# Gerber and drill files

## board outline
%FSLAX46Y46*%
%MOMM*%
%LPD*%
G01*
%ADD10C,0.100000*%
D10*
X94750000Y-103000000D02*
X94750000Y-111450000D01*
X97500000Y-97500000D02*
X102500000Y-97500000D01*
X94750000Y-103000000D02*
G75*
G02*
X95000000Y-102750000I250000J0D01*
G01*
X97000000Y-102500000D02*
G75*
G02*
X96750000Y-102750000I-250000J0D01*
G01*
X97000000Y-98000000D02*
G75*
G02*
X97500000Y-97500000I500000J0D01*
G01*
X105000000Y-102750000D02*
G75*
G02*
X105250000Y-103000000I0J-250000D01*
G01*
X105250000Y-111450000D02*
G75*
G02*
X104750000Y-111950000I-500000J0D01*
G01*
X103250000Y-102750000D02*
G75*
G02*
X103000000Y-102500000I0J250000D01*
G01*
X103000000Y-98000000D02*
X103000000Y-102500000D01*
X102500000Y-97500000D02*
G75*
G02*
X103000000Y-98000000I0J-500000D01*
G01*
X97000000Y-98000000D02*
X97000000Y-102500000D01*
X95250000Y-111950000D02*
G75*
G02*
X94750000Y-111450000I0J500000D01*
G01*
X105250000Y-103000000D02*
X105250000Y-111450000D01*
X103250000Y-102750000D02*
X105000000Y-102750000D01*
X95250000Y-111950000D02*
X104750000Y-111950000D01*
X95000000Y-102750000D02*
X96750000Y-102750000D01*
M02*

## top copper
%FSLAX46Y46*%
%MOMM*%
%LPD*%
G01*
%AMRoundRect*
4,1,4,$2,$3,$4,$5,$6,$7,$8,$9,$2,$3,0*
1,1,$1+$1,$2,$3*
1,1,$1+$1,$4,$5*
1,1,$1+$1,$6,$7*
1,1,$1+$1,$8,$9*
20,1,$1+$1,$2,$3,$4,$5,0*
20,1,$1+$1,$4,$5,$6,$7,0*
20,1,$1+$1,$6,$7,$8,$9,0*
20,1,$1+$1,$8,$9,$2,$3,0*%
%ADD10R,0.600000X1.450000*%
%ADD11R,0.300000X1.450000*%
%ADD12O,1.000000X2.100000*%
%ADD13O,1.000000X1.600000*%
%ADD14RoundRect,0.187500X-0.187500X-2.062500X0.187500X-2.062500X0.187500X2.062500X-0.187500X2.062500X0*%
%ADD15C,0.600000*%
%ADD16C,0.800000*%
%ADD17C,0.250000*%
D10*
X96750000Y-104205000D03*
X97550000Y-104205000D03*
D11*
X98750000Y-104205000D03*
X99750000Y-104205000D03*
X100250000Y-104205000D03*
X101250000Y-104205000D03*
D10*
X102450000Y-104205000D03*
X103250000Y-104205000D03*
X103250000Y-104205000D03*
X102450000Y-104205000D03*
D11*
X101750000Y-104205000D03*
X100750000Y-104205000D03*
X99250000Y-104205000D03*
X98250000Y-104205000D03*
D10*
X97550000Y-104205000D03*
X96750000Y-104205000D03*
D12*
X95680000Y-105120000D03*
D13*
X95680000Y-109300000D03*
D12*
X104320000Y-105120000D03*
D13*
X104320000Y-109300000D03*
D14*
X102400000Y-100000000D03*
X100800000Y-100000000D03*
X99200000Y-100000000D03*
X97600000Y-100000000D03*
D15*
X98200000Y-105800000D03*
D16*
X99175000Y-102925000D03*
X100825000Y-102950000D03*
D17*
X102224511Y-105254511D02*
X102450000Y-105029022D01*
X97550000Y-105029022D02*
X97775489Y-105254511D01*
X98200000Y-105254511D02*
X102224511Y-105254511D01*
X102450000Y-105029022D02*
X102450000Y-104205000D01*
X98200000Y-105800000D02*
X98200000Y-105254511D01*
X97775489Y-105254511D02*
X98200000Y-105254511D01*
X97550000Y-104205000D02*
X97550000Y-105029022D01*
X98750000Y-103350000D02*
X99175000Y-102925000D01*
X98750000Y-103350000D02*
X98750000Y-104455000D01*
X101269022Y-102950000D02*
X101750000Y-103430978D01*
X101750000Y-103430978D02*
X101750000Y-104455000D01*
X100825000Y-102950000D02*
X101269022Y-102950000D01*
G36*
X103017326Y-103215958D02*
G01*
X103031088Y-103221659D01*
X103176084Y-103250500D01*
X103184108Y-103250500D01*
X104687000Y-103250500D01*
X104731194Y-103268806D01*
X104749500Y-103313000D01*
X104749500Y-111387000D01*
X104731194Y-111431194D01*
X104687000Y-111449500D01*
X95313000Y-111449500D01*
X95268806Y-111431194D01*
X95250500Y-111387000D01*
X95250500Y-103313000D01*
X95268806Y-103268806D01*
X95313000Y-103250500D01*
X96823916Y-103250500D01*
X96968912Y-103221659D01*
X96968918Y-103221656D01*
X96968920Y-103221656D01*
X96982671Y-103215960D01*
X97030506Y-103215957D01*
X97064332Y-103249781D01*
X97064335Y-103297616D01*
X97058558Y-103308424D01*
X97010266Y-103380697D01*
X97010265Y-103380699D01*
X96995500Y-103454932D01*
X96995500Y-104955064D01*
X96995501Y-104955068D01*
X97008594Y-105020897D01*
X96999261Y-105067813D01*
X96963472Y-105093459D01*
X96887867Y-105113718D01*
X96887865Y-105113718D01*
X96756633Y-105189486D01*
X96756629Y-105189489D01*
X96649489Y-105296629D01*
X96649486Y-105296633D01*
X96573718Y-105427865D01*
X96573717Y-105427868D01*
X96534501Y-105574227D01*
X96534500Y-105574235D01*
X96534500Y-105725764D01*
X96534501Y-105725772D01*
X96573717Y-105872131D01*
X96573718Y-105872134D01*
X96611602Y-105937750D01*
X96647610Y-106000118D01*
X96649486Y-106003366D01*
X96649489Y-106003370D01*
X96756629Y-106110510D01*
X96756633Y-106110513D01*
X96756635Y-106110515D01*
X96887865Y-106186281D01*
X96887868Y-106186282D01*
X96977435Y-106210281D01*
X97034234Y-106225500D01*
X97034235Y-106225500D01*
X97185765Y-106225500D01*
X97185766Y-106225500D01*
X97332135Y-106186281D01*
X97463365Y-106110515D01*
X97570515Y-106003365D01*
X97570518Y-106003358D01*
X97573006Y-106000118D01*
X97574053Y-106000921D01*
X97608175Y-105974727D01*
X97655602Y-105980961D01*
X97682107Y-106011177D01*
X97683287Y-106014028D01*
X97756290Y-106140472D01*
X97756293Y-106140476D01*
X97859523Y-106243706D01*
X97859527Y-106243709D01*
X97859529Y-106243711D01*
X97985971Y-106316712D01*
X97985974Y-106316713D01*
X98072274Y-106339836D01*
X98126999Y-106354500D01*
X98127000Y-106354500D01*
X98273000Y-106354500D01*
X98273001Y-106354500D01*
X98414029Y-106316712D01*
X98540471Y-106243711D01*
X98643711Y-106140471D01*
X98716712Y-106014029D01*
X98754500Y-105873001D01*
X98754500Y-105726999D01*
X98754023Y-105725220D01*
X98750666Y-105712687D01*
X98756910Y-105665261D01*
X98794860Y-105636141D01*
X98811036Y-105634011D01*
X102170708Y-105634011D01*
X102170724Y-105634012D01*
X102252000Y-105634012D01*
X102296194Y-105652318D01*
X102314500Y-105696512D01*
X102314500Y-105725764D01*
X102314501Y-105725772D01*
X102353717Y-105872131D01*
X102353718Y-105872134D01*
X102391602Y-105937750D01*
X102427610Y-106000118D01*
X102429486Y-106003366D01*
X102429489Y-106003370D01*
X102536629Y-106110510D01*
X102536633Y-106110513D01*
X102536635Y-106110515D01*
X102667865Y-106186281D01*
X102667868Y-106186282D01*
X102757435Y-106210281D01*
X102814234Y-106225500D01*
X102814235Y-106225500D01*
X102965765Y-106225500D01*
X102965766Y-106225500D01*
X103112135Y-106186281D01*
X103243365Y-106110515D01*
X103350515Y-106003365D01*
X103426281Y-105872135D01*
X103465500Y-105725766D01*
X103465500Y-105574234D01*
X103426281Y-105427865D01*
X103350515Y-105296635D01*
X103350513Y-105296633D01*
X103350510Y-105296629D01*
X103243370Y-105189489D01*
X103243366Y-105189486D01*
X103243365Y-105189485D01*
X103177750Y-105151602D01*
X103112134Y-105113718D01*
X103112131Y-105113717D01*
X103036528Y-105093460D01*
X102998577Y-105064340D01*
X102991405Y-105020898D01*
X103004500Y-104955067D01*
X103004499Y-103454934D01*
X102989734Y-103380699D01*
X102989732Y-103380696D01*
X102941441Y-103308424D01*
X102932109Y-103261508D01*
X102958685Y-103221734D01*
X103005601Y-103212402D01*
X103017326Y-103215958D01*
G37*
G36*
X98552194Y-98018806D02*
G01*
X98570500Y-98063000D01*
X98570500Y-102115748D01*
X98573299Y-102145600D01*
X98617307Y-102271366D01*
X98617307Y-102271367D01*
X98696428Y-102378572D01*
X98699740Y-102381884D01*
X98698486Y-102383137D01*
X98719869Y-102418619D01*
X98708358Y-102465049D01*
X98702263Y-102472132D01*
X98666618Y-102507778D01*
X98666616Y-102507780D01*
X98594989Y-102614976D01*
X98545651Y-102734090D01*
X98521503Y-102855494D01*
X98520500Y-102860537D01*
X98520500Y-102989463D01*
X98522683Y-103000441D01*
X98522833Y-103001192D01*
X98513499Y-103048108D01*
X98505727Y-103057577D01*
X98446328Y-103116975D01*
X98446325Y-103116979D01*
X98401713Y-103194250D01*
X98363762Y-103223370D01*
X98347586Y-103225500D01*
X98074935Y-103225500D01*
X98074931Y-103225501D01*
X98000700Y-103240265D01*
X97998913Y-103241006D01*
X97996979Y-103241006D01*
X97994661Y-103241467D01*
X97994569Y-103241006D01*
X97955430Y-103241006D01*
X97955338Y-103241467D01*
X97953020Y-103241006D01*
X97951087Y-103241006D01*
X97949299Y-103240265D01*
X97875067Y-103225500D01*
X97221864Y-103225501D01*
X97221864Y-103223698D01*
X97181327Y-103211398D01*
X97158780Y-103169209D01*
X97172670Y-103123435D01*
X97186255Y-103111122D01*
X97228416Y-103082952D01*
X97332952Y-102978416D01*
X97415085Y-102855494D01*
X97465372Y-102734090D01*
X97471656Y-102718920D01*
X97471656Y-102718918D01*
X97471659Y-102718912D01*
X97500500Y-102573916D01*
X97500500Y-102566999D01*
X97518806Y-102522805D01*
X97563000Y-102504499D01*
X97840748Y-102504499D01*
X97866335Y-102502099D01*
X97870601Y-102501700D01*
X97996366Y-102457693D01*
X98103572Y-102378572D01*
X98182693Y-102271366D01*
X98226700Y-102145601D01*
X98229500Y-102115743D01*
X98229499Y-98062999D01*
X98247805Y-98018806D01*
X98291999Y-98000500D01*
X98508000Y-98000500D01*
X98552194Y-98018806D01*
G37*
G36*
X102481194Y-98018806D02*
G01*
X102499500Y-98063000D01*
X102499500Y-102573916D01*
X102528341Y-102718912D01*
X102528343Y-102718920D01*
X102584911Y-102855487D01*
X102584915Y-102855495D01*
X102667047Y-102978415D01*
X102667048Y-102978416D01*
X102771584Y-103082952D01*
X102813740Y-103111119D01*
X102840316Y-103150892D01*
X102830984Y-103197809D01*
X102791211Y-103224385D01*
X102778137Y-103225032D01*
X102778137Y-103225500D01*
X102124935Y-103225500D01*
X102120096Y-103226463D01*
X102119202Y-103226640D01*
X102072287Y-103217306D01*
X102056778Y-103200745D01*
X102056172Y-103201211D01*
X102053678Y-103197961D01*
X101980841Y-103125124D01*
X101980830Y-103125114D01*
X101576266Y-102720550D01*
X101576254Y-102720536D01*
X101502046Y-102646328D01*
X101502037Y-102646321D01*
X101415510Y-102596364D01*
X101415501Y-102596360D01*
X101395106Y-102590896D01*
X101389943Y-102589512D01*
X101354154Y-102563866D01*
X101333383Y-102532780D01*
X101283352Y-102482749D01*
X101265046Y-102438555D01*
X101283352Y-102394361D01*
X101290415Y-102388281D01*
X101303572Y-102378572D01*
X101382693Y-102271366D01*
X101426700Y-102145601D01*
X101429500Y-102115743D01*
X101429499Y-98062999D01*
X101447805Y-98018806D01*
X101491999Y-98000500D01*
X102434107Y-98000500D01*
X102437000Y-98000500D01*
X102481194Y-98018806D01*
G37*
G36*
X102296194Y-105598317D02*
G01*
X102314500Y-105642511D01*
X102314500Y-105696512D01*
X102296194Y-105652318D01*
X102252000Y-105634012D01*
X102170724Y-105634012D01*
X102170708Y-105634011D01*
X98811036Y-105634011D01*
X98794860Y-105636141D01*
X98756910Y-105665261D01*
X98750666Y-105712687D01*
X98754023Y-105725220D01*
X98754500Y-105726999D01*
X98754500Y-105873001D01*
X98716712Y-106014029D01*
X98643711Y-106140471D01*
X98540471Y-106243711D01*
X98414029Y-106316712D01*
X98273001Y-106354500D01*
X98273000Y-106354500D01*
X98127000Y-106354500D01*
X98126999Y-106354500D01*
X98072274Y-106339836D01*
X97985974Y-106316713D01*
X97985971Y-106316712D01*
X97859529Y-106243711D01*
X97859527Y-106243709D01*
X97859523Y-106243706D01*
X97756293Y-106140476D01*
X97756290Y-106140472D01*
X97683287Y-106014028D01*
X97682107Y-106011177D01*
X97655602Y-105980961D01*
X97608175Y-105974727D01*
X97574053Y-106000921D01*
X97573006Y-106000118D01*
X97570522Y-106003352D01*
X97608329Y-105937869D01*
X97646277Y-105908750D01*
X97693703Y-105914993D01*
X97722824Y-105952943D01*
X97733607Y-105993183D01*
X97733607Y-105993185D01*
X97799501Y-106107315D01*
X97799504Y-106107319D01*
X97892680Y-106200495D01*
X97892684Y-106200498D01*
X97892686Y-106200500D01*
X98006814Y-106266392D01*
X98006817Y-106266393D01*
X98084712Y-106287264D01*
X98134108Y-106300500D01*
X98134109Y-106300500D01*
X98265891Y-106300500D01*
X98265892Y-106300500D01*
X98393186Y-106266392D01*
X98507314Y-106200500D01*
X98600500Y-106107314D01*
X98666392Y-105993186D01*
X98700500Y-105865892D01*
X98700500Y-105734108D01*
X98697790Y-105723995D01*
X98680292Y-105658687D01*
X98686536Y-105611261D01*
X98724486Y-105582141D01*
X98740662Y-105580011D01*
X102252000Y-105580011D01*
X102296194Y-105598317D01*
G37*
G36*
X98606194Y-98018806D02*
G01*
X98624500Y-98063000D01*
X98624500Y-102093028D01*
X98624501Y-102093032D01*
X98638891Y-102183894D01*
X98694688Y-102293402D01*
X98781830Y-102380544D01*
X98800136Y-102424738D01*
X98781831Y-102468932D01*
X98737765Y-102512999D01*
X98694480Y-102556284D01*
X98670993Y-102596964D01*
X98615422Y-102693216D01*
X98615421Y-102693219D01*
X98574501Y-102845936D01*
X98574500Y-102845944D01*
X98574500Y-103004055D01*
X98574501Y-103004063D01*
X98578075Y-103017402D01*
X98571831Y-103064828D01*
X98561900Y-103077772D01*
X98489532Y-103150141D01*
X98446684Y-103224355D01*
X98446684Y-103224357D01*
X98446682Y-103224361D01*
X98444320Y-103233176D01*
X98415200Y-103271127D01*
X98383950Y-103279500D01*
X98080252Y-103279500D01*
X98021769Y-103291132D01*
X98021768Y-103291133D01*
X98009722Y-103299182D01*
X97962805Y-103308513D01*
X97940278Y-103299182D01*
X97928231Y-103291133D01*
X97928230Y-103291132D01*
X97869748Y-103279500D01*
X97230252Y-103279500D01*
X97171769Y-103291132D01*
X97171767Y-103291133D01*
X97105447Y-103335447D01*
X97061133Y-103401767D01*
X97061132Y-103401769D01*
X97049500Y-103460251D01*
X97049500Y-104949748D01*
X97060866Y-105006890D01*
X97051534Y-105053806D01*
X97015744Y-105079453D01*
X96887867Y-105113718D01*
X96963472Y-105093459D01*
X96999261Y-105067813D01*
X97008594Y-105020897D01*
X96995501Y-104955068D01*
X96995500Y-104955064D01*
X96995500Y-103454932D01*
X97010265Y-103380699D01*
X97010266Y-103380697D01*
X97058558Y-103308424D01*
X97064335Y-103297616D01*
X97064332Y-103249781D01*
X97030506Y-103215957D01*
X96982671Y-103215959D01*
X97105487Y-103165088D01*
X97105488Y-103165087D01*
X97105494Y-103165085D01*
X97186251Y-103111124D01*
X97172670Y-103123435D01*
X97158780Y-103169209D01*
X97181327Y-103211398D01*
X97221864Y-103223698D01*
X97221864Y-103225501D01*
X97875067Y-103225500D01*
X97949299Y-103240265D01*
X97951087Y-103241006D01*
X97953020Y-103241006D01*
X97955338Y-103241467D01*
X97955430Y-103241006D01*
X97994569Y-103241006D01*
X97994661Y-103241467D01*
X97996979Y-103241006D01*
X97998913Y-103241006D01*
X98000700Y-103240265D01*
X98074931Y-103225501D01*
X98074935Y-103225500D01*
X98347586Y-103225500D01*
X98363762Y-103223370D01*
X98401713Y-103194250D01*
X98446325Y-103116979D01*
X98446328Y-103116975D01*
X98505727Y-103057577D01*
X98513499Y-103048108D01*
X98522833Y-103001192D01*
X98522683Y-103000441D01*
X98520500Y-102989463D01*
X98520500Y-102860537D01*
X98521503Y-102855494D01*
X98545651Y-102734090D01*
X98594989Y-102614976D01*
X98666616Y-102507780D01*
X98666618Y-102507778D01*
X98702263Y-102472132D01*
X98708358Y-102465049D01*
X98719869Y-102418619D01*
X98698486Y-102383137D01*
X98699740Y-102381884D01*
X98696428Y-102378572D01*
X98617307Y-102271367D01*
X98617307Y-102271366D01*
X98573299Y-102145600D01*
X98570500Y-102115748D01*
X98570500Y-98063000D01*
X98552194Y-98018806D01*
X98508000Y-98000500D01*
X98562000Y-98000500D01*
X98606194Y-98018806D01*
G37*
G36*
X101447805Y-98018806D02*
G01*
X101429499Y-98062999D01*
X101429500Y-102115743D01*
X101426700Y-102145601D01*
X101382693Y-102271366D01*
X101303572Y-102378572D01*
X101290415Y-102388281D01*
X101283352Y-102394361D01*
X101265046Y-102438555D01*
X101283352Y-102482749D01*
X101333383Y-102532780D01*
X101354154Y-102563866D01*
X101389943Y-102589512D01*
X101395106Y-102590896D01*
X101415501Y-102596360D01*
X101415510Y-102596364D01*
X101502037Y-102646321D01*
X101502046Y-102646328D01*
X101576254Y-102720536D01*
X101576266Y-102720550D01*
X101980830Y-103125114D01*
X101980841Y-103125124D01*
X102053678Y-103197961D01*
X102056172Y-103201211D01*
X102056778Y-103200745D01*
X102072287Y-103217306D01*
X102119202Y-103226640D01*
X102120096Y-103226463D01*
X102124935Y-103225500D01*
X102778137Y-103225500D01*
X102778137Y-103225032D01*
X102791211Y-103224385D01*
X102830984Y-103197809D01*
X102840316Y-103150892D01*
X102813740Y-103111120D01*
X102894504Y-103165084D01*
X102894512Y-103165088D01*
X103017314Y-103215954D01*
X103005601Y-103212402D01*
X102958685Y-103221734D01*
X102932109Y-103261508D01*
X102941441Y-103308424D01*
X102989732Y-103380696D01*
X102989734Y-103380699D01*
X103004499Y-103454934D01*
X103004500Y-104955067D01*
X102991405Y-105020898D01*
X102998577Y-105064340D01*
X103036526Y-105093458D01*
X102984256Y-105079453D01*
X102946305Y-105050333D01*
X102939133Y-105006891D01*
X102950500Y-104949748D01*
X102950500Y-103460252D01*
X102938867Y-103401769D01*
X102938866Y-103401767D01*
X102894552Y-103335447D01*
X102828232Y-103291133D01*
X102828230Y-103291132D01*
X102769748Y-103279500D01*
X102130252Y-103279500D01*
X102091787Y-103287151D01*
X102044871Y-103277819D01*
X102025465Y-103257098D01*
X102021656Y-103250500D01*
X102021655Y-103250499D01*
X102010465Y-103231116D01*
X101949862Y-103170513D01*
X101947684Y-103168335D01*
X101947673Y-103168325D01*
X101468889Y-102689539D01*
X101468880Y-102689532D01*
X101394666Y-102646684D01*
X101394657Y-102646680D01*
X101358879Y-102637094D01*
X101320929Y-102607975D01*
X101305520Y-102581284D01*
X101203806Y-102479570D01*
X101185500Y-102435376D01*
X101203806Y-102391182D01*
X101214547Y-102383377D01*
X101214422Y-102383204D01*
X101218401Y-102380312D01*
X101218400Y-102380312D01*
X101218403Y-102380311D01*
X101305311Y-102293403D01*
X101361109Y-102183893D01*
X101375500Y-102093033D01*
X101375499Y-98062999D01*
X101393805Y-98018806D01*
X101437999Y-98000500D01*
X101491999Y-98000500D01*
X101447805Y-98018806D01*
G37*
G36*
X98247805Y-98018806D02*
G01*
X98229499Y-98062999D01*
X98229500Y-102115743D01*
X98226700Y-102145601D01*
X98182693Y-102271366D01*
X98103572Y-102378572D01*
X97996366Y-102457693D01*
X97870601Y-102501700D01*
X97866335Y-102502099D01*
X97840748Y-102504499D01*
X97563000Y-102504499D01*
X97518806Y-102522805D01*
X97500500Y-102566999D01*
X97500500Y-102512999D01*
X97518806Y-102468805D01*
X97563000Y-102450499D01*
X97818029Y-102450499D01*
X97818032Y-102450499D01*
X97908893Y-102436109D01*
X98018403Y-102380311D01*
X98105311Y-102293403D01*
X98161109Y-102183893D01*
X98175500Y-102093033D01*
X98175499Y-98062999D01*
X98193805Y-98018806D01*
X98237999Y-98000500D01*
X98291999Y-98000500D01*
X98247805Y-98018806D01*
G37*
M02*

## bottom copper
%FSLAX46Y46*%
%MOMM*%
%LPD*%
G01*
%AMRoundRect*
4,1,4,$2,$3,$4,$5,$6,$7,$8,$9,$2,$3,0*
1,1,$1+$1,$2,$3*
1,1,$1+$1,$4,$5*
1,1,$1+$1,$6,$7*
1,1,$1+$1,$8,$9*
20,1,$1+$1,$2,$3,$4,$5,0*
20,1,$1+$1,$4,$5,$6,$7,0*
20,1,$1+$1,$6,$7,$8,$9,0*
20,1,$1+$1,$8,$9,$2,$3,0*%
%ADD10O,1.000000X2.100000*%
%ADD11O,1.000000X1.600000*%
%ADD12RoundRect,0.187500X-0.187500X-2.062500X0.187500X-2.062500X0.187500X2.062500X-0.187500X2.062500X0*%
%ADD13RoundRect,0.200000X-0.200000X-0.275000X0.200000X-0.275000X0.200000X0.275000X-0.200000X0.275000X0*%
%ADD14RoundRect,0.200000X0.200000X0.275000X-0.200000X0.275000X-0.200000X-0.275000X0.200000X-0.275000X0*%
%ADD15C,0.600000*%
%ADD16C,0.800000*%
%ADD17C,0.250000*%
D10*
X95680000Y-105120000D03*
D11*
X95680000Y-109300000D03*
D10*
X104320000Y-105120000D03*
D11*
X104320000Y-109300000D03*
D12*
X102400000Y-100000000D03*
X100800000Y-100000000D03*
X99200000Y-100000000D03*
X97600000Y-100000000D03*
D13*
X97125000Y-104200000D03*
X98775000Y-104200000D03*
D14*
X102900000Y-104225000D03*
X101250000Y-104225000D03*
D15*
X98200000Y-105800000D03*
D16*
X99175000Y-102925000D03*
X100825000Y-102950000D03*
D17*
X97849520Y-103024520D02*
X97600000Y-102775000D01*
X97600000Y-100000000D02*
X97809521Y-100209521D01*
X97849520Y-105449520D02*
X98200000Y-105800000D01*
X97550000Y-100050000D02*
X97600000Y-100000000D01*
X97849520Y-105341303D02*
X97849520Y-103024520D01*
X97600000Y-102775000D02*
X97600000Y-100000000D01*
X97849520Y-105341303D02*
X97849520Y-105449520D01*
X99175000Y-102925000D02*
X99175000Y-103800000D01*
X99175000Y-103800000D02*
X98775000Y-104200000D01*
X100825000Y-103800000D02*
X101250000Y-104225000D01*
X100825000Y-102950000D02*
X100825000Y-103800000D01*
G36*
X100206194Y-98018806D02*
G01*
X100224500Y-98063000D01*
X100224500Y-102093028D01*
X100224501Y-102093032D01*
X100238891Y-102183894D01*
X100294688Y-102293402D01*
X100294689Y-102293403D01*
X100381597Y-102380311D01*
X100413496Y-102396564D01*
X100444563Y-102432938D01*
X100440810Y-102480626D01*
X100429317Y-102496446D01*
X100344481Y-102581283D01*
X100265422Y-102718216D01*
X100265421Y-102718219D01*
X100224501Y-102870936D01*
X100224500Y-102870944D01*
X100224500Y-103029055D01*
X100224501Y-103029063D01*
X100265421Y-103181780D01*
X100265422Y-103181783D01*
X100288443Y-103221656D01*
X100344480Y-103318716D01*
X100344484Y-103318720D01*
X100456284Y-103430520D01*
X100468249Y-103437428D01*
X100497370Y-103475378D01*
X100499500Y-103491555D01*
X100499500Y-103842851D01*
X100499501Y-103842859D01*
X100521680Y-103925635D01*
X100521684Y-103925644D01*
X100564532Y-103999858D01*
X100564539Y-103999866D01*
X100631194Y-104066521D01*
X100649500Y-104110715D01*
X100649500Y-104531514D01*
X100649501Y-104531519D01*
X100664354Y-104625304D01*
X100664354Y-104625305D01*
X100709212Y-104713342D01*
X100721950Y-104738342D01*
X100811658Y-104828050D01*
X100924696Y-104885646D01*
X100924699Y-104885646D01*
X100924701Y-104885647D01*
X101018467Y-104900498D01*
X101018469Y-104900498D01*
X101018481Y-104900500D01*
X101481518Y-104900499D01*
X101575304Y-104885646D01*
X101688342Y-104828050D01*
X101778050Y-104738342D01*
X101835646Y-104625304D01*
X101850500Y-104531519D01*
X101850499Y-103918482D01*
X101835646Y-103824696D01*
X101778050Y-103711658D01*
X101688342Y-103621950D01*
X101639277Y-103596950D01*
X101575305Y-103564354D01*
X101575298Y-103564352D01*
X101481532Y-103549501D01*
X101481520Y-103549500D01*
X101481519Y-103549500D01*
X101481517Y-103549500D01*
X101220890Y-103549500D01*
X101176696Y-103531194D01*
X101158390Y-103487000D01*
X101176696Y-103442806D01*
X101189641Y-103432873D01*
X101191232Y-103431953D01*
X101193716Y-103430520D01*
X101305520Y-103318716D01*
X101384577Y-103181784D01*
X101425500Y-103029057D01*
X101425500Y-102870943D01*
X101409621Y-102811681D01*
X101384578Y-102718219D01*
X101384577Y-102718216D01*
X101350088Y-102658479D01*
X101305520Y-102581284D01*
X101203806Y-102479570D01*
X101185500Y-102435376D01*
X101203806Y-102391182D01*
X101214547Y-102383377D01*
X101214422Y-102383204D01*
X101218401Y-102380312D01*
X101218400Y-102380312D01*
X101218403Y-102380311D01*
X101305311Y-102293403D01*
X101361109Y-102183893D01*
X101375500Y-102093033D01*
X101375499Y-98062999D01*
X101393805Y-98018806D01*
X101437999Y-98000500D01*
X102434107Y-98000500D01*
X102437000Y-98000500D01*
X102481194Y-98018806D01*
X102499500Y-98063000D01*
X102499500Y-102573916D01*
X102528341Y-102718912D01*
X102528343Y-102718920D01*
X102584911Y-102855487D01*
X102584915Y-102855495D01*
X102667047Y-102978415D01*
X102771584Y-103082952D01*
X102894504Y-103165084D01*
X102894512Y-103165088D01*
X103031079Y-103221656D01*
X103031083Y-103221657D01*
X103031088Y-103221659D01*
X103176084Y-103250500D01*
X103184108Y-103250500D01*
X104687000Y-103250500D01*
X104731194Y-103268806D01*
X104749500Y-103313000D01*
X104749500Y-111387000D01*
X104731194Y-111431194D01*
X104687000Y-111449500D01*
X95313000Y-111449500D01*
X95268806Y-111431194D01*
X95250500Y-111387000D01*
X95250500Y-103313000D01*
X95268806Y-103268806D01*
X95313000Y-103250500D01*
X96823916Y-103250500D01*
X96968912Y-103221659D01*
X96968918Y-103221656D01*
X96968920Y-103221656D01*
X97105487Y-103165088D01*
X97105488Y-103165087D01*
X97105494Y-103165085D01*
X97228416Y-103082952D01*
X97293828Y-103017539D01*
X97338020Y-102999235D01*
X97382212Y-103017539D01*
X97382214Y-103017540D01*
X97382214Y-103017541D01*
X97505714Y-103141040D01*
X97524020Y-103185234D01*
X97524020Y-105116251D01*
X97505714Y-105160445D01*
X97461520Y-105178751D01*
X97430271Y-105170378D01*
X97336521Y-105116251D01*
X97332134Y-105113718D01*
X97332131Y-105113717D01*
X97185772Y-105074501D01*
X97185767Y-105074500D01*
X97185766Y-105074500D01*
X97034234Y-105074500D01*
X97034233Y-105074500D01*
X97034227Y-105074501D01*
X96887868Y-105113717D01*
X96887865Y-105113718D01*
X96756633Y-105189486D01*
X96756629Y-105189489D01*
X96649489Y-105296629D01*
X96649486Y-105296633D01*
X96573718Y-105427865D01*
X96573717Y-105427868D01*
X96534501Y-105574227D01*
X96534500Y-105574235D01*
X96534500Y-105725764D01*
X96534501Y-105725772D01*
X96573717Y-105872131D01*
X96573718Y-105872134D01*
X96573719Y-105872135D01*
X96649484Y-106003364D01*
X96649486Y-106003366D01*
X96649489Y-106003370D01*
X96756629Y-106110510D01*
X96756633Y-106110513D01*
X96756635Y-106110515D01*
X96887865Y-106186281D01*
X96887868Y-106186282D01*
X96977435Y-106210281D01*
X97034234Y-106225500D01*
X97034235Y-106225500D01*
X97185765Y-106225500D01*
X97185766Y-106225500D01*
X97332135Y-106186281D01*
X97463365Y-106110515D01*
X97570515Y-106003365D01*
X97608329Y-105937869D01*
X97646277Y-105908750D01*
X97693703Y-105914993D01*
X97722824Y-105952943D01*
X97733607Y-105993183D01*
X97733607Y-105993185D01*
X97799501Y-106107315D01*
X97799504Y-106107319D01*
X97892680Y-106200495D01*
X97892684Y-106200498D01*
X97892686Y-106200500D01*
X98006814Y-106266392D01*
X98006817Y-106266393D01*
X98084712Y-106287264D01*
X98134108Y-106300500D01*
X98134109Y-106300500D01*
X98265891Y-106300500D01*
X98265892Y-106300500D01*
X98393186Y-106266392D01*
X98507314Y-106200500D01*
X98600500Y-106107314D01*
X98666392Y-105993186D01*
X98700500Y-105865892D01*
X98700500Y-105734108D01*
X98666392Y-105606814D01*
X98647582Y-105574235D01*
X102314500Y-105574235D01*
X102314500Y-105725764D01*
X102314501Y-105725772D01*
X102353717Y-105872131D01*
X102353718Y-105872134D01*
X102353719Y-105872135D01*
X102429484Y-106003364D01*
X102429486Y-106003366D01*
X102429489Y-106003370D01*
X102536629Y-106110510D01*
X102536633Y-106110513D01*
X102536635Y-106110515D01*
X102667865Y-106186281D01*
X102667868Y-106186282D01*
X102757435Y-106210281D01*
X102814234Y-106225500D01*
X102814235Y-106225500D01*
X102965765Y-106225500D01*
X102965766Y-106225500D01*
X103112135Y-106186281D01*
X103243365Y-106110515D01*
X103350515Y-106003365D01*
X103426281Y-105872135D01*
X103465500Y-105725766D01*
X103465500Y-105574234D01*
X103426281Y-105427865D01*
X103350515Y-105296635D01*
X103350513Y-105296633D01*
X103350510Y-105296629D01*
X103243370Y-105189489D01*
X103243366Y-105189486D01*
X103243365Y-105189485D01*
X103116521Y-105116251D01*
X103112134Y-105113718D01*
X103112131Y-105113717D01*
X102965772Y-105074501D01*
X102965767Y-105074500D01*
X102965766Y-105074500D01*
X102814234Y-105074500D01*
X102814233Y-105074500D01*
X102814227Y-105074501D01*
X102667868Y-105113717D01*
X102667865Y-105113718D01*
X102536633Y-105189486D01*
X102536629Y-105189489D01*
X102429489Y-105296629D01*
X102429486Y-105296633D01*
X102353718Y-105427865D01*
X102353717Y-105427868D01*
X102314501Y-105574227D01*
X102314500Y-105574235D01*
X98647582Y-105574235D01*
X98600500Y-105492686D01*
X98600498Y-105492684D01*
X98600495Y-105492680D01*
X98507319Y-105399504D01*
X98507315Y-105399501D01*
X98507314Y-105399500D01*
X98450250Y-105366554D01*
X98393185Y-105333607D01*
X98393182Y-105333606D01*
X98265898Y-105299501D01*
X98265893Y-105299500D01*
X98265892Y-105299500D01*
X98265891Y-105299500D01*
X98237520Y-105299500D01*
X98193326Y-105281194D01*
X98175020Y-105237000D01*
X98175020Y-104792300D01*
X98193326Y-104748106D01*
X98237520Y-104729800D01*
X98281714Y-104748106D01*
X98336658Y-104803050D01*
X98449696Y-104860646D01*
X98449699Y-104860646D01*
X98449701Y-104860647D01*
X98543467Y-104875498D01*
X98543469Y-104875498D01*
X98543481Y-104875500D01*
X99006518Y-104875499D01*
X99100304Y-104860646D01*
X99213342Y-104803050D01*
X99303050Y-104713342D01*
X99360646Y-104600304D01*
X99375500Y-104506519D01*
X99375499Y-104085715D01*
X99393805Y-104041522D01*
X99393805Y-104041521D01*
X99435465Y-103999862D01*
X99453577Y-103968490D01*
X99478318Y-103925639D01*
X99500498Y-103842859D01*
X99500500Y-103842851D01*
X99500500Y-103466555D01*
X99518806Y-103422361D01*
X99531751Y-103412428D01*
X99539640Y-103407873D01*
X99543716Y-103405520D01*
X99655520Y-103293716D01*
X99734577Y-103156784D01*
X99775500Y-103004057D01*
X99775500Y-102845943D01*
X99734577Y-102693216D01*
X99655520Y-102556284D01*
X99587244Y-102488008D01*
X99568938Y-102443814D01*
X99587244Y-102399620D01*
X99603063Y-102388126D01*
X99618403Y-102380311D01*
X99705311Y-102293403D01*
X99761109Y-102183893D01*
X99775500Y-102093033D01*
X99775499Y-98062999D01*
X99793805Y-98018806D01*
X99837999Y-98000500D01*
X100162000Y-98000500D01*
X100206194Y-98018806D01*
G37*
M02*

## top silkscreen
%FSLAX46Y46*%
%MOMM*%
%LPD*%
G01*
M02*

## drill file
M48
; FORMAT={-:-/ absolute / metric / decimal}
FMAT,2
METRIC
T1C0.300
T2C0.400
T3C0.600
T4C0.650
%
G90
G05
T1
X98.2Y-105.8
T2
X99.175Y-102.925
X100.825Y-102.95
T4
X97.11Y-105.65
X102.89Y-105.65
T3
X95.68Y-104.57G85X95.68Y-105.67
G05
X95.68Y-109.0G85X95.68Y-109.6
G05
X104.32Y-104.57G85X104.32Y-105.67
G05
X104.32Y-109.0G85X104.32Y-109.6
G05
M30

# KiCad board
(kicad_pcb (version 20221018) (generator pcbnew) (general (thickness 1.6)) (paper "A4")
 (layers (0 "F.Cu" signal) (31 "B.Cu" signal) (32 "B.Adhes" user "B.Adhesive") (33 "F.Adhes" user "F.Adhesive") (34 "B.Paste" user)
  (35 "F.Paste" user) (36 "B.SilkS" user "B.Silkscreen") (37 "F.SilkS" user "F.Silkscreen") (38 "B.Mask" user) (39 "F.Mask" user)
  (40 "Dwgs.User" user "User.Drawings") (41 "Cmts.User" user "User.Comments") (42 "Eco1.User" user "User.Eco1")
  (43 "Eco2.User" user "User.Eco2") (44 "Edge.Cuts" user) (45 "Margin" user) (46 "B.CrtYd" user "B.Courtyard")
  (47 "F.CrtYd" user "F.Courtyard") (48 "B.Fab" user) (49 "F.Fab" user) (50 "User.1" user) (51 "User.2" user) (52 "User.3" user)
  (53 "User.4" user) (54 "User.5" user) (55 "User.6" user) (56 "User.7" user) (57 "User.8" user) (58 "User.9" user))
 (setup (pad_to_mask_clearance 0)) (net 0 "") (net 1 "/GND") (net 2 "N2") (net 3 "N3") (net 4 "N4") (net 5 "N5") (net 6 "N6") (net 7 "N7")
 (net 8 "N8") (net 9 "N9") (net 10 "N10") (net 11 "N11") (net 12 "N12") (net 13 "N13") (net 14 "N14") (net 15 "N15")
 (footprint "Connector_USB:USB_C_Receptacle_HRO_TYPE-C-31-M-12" (layer "F.Cu") (at 100 108.25)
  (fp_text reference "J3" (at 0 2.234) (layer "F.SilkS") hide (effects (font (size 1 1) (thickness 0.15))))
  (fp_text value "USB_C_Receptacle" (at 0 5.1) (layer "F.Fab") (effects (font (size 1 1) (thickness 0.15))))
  (pad "" np_thru_hole circle (at -2.89 -2.6) (size 0.65 0.65) (drill 0.65) (layers "*.Cu" "*.Mask"))
  (pad "" np_thru_hole circle (at 2.89 -2.6) (size 0.65 0.65) (drill 0.65) (layers "*.Cu" "*.Mask"))
  (pad "A1" smd rect (at -3.25 -4.045) (size 0.6 1.45) (layers "F.Cu" "F.Paste" "F.Mask") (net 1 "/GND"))
  (pad "A4" smd rect (at -2.45 -4.045) (size 0.6 1.45) (layers "F.Cu" "F.Paste" "F.Mask") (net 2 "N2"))
  (pad "A5" smd rect (at -1.25 -4.045) (size 0.3 1.45) (layers "F.Cu" "F.Paste" "F.Mask") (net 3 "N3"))
  (pad "A6" smd rect (at -0.25 -4.045) (size 0.3 1.45) (layers "F.Cu" "F.Paste" "F.Mask") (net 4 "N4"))
  (pad "A7" smd rect (at 0.25 -4.045) (size 0.3 1.45) (layers "F.Cu" "F.Paste" "F.Mask") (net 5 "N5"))
  (pad "A8" smd rect (at 1.25 -4.045) (size 0.3 1.45) (layers "F.Cu" "F.Paste" "F.Mask") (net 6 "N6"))
  (pad "A9" smd rect (at 2.45 -4.045) (size 0.6 1.45) (layers "F.Cu" "F.Paste" "F.Mask") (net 2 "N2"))
  (pad "A12" smd rect (at 3.25 -4.045) (size 0.6 1.45) (layers "F.Cu" "F.Paste" "F.Mask") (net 1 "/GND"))
  (pad "B1" smd rect (at 3.25 -4.045) (size 0.6 1.45) (layers "F.Cu" "F.Paste" "F.Mask") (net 1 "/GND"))
  (pad "B4" smd rect (at 2.45 -4.045) (size 0.6 1.45) (layers "F.Cu" "F.Paste" "F.Mask") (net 2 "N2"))
  (pad "B5" smd rect (at 1.75 -4.045) (size 0.3 1.45) (layers "F.Cu" "F.Paste" "F.Mask") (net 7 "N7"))
  (pad "B6" smd rect (at 0.75 -4.045) (size 0.3 1.45) (layers "F.Cu" "F.Paste" "F.Mask") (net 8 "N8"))
  (pad "B7" smd rect (at -0.75 -4.045) (size 0.3 1.45) (layers "F.Cu" "F.Paste" "F.Mask") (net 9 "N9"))
  (pad "B8" smd rect (at -1.75 -4.045) (size 0.3 1.45) (layers "F.Cu" "F.Paste" "F.Mask") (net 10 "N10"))
  (pad "B9" smd rect (at -2.45 -4.045) (size 0.6 1.45) (layers "F.Cu" "F.Paste" "F.Mask") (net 2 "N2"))
  (pad "B12" smd rect (at -3.25 -4.045) (size 0.6 1.45) (layers "F.Cu" "F.Paste" "F.Mask") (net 1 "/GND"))
  (pad "S1" thru_hole oval (at -4.32 -3.13) (size 1 2.1) (drill oval 0.6 1.7) (layers "*.Cu" "*.Mask") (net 1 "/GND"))
  (pad "S1" thru_hole oval (at -4.32 1.05) (size 1 1.6) (drill oval 0.6 1.2) (layers "*.Cu" "*.Mask") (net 1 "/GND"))
  (pad "S1" thru_hole oval (at 4.32 -3.13) (size 1 2.1) (drill oval 0.6 1.7) (layers "*.Cu" "*.Mask") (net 1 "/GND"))
  (pad "S1" thru_hole oval (at 4.32 1.05) (size 1 1.6) (drill oval 0.6 1.2) (layers "*.Cu" "*.Mask") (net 1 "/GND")))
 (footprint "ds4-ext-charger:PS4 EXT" (layer "F.Cu") (at 100 100)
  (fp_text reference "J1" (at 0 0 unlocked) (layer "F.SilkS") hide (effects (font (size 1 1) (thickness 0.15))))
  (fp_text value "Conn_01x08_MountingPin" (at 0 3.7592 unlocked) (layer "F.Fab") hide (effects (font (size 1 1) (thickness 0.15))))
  (pad "6" smd roundrect (at 2.4 0) (size 0.75 4.5) (layers "B.Cu" "B.Paste" "B.Mask") (roundrect_rratio 0.25) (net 1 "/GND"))
  (pad "7" smd roundrect (at 2.4 0) (size 0.75 4.5) (layers "F.Cu" "F.Paste" "F.Mask") (roundrect_rratio 0.25) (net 1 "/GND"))
  (pad "8" smd roundrect (at 0.8 0) (size 0.75 4.5) (layers "B.Cu" "B.Paste" "B.Mask") (roundrect_rratio 0.25) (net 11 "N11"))
  (pad "9" smd roundrect (at 0.8 0) (size 0.75 4.5) (layers "F.Cu" "F.Paste" "F.Mask") (roundrect_rratio 0.25) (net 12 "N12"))
  (pad "10" smd roundrect (at -0.8 0) (size 0.75 4.5) (layers "B.Cu" "B.Paste" "B.Mask") (roundrect_rratio 0.25) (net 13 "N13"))
  (pad "11" smd roundrect (at -0.8 0) (size 0.75 4.5) (layers "F.Cu" "F.Paste" "F.Mask") (roundrect_rratio 0.25) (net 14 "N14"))
  (pad "12" smd roundrect (at -2.4 0) (size 0.75 4.5) (layers "B.Cu" "B.Paste" "B.Mask") (roundrect_rratio 0.25) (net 2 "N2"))
  (pad "13" smd roundrect (at -2.4 0) (size 0.75 4.5) (layers "F.Cu" "F.Paste" "F.Mask") (roundrect_rratio 0.25) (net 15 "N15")))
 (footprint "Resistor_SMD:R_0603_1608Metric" (layer "B.Cu") (at 97.95 104.2)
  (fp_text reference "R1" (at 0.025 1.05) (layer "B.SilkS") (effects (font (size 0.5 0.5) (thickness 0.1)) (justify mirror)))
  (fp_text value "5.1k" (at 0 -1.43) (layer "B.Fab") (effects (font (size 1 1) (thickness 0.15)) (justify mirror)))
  (pad "1" smd roundrect (at -0.825 0) (size 0.8 0.95) (layers "B.Cu" "B.Paste" "B.Mask") (roundrect_rratio 0.25) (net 1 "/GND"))
  (pad "2" smd roundrect (at 0.825 0) (size 0.8 0.95) (layers "B.Cu" "B.Paste" "B.Mask") (roundrect_rratio 0.25) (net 3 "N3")))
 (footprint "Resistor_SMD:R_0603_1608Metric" (layer "B.Cu") (at 102.075 104.225 180)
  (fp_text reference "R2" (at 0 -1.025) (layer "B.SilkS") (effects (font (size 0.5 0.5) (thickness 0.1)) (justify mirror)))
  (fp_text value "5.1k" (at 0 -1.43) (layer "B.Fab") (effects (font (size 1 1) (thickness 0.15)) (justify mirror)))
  (pad "1" smd roundrect (at -0.825 0 180) (size 0.8 0.95) (layers "B.Cu" "B.Paste" "B.Mask") (roundrect_rratio 0.25) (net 1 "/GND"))
  (pad "2" smd roundrect (at 0.825 0 180) (size 0.8 0.95) (layers "B.Cu" "B.Paste" "B.Mask") (roundrect_rratio 0.25) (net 7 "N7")))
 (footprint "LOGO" (layer "B.Cu") (at 100 106 180)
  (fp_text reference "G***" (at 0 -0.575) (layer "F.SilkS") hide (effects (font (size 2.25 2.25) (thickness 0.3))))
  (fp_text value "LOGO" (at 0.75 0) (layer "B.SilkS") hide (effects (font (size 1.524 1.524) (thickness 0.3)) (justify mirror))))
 (gr_line (start 94.75 103) (end 94.75 111.45) (stroke (width 0.1) (type solid)) (layer "Edge.Cuts"))
 (gr_line (start 97.5 97.5) (end 102.5 97.5) (stroke (width 0.1) (type solid)) (layer "Edge.Cuts"))
 (gr_arc (start 94.75 103) (mid 94.823223 102.823223) (end 95 102.75) (stroke (width 0.1) (type solid)) (layer "Edge.Cuts"))
 (gr_arc (start 97 102.5) (mid 96.926777 102.676777) (end 96.75 102.75) (stroke (width 0.1) (type solid)) (layer "Edge.Cuts"))
 (gr_arc (start 97 98) (mid 97.146447 97.646447) (end 97.5 97.5) (stroke (width 0.1) (type solid)) (layer "Edge.Cuts"))
 (gr_arc (start 105 102.75) (mid 105.176777 102.823223) (end 105.25 103) (stroke (width 0.1) (type solid)) (layer "Edge.Cuts"))
 (gr_arc (start 105.25 111.45) (mid 105.103553 111.803553) (end 104.75 111.95) (stroke (width 0.1) (type solid)) (layer "Edge.Cuts"))
 (gr_arc (start 103.25 102.75) (mid 103.073223 102.676777) (end 103 102.5) (stroke (width 0.1) (type solid)) (layer "Edge.Cuts"))
 (gr_line (start 103 98) (end 103 102.5) (stroke (width 0.1) (type solid)) (layer "Edge.Cuts"))
 (gr_arc (start 102.5 97.5) (mid 102.853553 97.646447) (end 103 98) (stroke (width 0.1) (type solid)) (layer "Edge.Cuts"))
 (gr_line (start 97 98) (end 97 102.5) (stroke (width 0.1) (type solid)) (layer "Edge.Cuts"))
 (gr_arc (start 95.25 111.95) (mid 94.896447 111.803553) (end 94.75 111.45) (stroke (width 0.1) (type solid)) (layer "Edge.Cuts"))
 (gr_line (start 105.25 103) (end 105.25 111.45) (stroke (width 0.1) (type solid)) (layer "Edge.Cuts"))
 (gr_line (start 103.25 102.75) (end 105 102.75) (stroke (width 0.1) (type solid)) (layer "Edge.Cuts"))
 (gr_line (start 95.25 111.95) (end 104.75 111.95) (stroke (width 0.1) (type solid)) (layer "Edge.Cuts"))
 (gr_line (start 95 102.75) (end 96.75 102.75) (stroke (width 0.1) (type solid)) (layer "Edge.Cuts"))
 (segment (start 102.224511 105.254511) (end 102.45 105.029022) (width 0.25) (layer "F.Cu") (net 2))
 (segment (start 97.55 105.029022) (end 97.775489 105.254511) (width 0.25) (layer "F.Cu") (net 2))
 (segment (start 98.2 105.254511) (end 102.224511 105.254511) (width 0.25) (layer "F.Cu") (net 2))
 (segment (start 102.45 105.029022) (end 102.45 104.205) (width 0.25) (layer "F.Cu") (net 2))
 (segment (start 98.2 105.8) (end 98.2 105.254511) (width 0.25) (layer "F.Cu") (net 2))
 (segment (start 97.775489 105.254511) (end 98.2 105.254511) (width 0.25) (layer "F.Cu") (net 2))
 (segment (start 97.55 104.205) (end 97.55 105.029022) (width 0.25) (layer "F.Cu") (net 2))
 (via (at 98.2 105.8) (size 0.6) (drill 0.3) (layers "F.Cu" "B.Cu") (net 2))
 (segment (start 97.84952 103.02452) (end 97.6 102.775) (width 0.25) (layer "B.Cu") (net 2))
 (segment (start 97.6 100) (end 97.809521 100.209521) (width 0.25) (layer "B.Cu") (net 2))
 (segment (start 97.84952 105.44952) (end 98.2 105.8) (width 0.25) (layer "B.Cu") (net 2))
 (segment (start 97.55 100.05) (end 97.6 100) (width 0.25) (layer "B.Cu") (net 2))
 (segment (start 97.84952 105.341303) (end 97.84952 103.02452) (width 0.25) (layer "B.Cu") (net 2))
 (segment (start 97.6 102.775) (end 97.6 100) (width 0.25) (layer "B.Cu") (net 2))
 (segment (start 97.84952 105.341303) (end 97.84952 105.44952) (width 0.25) (layer "B.Cu") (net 2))
 (segment (start 98.75 103.35) (end 99.175 102.925) (width 0.25) (layer "F.Cu") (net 3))
 (segment (start 98.75 103.35) (end 98.75 104.455) (width 0.25) (layer "F.Cu") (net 3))
 (via (at 99.175 102.925) (size 0.8) (drill 0.4) (layers "F.Cu" "B.Cu") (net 3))
 (segment (start 99.175 102.925) (end 99.175 103.8) (width 0.25) (layer "B.Cu") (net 3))
 (segment (start 99.175 103.8) (end 98.775 104.2) (width 0.25) (layer "B.Cu") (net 3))
 (segment (start 101.269022 102.95) (end 101.75 103.430978) (width 0.25) (layer "F.Cu") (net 7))
 (segment (start 101.75 103.430978) (end 101.75 104.455) (width 0.25) (layer "F.Cu") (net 7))
 (segment (start 100.825 102.95) (end 101.269022 102.95) (width 0.25) (layer "F.Cu") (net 7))
 (via (at 100.825 102.95) (size 0.8) (drill 0.4) (layers "F.Cu" "B.Cu") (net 7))
 (segment (start 100.825 103.8) (end 101.25 104.225) (width 0.25) (layer "B.Cu") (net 7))
 (segment (start 100.825 102.95) (end 100.825 103.8) (width 0.25) (layer "B.Cu") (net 7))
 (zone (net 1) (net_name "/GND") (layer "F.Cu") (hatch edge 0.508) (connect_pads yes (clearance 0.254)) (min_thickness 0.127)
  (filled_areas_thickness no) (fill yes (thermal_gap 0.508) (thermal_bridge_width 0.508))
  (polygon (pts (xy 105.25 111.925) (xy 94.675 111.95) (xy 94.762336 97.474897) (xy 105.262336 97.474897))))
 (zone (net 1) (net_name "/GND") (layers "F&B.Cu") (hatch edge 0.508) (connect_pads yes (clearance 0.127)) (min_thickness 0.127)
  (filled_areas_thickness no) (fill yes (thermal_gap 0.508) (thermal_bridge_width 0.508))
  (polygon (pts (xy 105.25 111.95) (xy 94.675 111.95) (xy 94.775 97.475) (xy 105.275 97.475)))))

